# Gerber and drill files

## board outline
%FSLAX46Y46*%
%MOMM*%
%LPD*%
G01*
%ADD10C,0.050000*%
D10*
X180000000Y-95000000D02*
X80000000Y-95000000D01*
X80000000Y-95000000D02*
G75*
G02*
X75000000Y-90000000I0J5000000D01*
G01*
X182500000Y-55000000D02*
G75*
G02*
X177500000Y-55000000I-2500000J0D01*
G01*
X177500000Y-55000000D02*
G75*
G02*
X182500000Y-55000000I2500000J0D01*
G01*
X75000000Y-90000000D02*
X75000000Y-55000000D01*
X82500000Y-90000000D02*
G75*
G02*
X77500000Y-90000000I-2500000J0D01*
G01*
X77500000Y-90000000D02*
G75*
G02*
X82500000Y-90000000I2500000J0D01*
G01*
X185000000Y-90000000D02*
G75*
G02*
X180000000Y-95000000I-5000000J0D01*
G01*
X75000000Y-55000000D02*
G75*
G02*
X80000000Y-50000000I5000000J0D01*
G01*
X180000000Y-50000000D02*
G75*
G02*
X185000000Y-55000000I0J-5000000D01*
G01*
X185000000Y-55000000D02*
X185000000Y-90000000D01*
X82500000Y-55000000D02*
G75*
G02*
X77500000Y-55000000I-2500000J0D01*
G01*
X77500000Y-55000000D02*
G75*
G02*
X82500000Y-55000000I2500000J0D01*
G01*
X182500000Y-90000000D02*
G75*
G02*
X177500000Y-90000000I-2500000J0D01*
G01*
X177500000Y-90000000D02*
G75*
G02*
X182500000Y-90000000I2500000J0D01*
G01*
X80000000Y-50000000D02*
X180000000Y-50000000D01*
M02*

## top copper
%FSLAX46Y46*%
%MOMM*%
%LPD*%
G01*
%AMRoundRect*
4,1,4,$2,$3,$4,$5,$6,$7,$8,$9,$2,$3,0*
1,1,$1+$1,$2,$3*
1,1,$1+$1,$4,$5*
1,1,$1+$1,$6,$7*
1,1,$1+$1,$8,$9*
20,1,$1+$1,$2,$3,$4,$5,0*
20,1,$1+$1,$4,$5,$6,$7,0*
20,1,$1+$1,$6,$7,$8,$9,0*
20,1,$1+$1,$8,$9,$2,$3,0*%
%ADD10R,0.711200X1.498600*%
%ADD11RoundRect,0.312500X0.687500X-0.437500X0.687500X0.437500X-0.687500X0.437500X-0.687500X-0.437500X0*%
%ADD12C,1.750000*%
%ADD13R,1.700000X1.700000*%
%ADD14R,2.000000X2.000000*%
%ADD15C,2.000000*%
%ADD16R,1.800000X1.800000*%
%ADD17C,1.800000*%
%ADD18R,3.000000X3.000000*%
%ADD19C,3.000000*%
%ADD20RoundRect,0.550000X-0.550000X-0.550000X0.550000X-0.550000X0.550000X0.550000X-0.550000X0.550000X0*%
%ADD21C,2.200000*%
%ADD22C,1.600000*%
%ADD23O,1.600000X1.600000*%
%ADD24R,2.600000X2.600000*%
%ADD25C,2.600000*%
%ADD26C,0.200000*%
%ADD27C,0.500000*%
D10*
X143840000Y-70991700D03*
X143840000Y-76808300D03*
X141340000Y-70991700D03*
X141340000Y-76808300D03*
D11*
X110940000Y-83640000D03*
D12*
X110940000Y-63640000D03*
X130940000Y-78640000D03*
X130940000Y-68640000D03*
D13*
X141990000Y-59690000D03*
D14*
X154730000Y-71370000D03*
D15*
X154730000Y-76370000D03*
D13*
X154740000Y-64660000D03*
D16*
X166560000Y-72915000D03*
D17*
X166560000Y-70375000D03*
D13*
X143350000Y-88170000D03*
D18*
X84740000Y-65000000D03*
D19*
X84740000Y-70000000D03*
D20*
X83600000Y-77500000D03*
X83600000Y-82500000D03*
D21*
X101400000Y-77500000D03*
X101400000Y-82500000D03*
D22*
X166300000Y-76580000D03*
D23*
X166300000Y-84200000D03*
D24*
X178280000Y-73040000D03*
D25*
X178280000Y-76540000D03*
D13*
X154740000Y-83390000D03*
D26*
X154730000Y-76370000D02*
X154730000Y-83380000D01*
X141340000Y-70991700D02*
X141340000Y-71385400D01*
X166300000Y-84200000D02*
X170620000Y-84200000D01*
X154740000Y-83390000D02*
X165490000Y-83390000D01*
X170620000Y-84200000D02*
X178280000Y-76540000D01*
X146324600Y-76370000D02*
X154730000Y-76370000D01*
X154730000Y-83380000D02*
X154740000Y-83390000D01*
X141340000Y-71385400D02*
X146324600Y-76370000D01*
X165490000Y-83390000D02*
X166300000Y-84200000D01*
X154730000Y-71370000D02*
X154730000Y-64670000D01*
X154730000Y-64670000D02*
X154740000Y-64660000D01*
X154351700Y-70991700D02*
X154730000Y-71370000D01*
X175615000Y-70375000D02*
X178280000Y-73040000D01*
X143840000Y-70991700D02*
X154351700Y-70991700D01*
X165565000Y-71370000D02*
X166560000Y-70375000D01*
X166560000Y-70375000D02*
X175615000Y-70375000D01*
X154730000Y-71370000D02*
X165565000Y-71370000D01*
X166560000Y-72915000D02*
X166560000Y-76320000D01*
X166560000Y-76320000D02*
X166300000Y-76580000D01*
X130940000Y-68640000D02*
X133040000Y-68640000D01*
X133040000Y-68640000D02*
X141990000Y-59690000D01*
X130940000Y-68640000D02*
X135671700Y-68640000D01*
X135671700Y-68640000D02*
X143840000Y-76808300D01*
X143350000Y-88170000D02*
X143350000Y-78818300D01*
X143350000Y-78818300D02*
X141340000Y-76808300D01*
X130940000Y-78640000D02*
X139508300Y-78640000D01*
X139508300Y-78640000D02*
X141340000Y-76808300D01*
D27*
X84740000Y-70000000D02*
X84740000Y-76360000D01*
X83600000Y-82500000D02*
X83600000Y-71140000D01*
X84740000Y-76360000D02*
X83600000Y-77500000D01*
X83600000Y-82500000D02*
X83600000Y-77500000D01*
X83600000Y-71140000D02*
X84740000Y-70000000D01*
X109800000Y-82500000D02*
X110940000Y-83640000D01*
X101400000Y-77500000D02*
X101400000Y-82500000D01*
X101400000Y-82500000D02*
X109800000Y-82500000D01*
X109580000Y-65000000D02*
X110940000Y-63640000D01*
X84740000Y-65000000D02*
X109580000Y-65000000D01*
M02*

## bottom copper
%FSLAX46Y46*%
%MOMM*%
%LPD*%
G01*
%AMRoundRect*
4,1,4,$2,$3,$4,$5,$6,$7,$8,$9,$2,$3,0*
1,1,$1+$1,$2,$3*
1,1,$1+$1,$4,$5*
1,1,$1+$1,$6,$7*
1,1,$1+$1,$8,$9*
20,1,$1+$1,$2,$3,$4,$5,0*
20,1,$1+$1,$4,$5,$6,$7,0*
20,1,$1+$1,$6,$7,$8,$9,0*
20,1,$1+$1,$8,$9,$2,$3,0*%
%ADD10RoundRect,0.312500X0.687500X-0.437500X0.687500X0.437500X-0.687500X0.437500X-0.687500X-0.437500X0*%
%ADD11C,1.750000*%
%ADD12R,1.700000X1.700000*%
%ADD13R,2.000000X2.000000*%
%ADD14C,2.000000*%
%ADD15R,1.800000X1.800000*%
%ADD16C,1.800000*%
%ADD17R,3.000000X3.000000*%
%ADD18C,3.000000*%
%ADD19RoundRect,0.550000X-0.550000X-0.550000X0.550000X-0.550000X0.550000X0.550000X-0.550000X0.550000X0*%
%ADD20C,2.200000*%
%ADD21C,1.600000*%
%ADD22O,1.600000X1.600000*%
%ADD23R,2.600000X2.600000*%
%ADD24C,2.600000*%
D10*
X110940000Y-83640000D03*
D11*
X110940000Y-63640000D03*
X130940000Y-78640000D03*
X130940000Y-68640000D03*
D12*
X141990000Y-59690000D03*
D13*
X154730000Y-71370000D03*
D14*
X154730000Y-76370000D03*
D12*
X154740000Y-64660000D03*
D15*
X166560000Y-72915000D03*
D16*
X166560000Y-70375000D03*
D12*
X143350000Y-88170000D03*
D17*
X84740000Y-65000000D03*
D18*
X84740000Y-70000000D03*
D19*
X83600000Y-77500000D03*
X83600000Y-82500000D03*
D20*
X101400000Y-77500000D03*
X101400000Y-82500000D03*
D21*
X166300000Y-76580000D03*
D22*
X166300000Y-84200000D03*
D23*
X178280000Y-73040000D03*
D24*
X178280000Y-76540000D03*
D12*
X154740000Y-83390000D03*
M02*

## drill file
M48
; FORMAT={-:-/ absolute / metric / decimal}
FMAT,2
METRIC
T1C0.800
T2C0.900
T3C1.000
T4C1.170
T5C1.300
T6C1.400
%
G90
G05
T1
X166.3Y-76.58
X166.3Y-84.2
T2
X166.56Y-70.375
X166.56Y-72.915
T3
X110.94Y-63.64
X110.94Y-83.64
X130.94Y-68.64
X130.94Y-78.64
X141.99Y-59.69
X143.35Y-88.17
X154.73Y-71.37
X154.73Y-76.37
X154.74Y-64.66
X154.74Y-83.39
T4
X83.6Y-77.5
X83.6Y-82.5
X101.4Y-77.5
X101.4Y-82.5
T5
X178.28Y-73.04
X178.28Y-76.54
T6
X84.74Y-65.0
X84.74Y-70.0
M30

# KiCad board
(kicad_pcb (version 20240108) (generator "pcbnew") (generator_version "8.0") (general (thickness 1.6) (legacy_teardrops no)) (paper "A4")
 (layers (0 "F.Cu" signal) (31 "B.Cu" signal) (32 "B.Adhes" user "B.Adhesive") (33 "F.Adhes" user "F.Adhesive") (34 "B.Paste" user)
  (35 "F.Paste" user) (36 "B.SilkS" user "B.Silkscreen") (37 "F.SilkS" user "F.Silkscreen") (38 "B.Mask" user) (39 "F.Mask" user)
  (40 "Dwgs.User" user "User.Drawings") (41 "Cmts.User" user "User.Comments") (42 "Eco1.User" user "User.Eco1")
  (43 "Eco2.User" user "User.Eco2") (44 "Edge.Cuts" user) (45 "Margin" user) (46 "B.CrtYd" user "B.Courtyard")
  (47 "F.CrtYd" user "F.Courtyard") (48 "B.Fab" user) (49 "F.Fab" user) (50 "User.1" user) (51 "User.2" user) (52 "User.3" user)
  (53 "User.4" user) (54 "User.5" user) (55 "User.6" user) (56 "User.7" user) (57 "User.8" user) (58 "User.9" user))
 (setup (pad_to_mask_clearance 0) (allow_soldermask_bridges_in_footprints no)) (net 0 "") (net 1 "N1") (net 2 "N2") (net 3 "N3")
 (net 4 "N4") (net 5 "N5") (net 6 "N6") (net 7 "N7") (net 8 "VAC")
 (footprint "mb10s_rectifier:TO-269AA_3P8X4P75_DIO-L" (layer "F.Cu") (at 142.59 73.9 -90)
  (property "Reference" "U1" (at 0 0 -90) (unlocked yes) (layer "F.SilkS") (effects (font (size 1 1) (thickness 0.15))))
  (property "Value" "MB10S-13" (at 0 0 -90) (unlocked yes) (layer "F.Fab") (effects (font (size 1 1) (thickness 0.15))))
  (pad "1" smd rect (at -2.9083 -1.25 270) (size 1.4986 0.7112) (layers "F.Cu" "F.Paste" "F.Mask") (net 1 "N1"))
  (pad "2" smd rect (at 2.9083 -1.25 270) (size 1.4986 0.7112) (layers "F.Cu" "F.Paste" "F.Mask") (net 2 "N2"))
  (pad "3" smd rect (at -2.9083 1.25 270) (size 1.4986 0.7112) (layers "F.Cu" "F.Paste" "F.Mask") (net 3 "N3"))
  (pad "4" smd rect (at 2.9083 1.25 270) (size 1.4986 0.7112) (layers "F.Cu" "F.Paste" "F.Mask") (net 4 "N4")))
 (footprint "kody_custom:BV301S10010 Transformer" (layer "F.Cu") (at 105.94 71.14 90)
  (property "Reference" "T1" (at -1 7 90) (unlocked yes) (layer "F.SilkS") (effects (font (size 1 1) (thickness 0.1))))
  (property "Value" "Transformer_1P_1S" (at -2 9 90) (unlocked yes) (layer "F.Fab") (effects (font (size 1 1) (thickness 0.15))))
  (pad "1" thru_hole roundrect (at -12.5 5 90) (size 1.5 2) (drill 1) (layers "*.Cu" "*.Mask") (remove_unused_layers no)
   (roundrect_rratio 0.2083333333) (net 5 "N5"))
  (pad "2" thru_hole circle (at 7.5 5 90) (size 1.75 1.75) (drill 1) (layers "*.Cu" "*.Mask") (remove_unused_layers no) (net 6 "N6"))
  (pad "3" thru_hole circle (at -7.5 25 90) (size 1.75 1.75) (drill 1) (layers "*.Cu" "*.Mask") (remove_unused_layers no) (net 4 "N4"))
  (pad "4" thru_hole circle (at 2.5 25 90) (size 1.75 1.75) (drill 1) (layers "*.Cu" "*.Mask") (remove_unused_layers no) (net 2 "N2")))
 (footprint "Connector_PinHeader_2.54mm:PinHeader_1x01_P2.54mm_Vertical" (layer "F.Cu") (at 141.99 59.69)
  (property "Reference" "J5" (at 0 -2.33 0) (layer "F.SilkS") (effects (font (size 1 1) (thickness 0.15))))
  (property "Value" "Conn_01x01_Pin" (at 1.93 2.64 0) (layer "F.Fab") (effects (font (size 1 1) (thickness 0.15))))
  (pad "1" thru_hole rect (at 0 0) (size 1.7 1.7) (drill 1) (layers "*.Cu" "*.Mask") (remove_unused_layers no) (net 2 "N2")))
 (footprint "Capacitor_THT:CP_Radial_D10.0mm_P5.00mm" (layer "F.Cu") (at 154.73 71.37 -90)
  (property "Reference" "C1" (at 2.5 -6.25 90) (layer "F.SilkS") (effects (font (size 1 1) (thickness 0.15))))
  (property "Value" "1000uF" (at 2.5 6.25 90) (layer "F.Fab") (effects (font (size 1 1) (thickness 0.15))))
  (pad "1" thru_hole rect (at 0 0 270) (size 2 2) (drill 1) (layers "*.Cu" "*.Mask") (remove_unused_layers no) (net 1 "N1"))
  (pad "2" thru_hole circle (at 5 0 270) (size 2 2) (drill 1) (layers "*.Cu" "*.Mask") (remove_unused_layers no) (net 3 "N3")))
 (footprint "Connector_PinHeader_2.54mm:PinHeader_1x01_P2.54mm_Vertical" (layer "F.Cu") (at 154.74 64.66)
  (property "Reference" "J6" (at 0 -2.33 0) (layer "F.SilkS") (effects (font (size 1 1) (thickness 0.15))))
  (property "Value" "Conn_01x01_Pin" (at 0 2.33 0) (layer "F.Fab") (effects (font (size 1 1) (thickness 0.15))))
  (pad "1" thru_hole rect (at 0 0) (size 1.7 1.7) (drill 1) (layers "*.Cu" "*.Mask") (remove_unused_layers no) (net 1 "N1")))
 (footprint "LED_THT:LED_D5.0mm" (layer "F.Cu") (at 166.56 72.915 90)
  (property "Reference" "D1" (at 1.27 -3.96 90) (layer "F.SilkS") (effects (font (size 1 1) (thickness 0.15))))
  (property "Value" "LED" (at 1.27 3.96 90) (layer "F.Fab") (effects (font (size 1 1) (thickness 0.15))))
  (pad "1" thru_hole rect (at 0 0 90) (size 1.8 1.8) (drill 0.9) (layers "*.Cu" "*.Mask") (remove_unused_layers no) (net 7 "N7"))
  (pad "2" thru_hole circle (at 2.54 0 90) (size 1.8 1.8) (drill 0.9) (layers "*.Cu" "*.Mask") (remove_unused_layers no) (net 1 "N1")))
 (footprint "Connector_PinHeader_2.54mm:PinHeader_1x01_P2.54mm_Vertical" (layer "F.Cu") (at 143.35 88.17)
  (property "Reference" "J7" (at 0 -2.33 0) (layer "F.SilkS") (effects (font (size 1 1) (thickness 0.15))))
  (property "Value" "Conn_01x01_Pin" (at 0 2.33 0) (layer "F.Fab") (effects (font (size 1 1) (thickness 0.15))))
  (pad "1" thru_hole rect (at 0 0) (size 1.7 1.7) (drill 1) (layers "*.Cu" "*.Mask") (remove_unused_layers no) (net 4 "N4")))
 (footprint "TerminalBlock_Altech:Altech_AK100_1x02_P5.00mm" (layer "F.Cu") (at 84.74 65 -90)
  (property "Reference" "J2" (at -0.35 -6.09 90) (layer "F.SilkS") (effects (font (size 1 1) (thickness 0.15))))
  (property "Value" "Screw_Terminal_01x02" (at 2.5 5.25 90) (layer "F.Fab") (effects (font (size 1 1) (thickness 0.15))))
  (pad "1" thru_hole rect (at 0 0 270) (size 3 3) (drill 1.4) (layers "*.Cu" "*.Mask") (remove_unused_layers no) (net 6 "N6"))
  (pad "2" thru_hole circle (at 5 0 270) (size 3 3) (drill 1.4) (layers "*.Cu" "*.Mask") (remove_unused_layers no) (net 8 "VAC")))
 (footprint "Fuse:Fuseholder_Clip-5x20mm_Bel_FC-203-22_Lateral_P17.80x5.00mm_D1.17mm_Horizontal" (layer "F.Cu") (at 83.6 77.5)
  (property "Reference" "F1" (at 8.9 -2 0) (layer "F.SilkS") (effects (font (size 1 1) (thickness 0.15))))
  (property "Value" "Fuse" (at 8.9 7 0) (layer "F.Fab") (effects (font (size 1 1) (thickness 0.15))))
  (pad "1" thru_hole roundrect (at 0 0) (size 2.2 2.2) (drill 1.17) (layers "*.Cu" "*.Mask") (remove_unused_layers no)
   (roundrect_rratio 0.25) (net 8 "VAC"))
  (pad "1" thru_hole roundrect (at 0 5) (size 2.2 2.2) (drill 1.17) (layers "*.Cu" "*.Mask") (remove_unused_layers no)
   (roundrect_rratio 0.25) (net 8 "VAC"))
  (pad "2" thru_hole circle (at 17.8 0) (size 2.2 2.2) (drill 1.17) (layers "*.Cu" "*.Mask") (remove_unused_layers no) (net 5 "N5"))
  (pad "2" thru_hole circle (at 17.8 5) (size 2.2 2.2) (drill 1.17) (layers "*.Cu" "*.Mask") (remove_unused_layers no) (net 5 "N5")))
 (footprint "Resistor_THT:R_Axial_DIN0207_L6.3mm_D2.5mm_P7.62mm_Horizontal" (layer "F.Cu") (at 166.3 76.58 -90)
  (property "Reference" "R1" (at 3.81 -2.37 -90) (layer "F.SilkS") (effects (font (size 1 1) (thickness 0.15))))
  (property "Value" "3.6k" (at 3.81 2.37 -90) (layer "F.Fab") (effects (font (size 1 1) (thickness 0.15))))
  (pad "1" thru_hole circle (at 0 0 270) (size 1.6 1.6) (drill 0.8) (layers "*.Cu" "*.Mask") (remove_unused_layers no) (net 7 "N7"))
  (pad "2" thru_hole oval (at 7.62 0 270) (size 1.6 1.6) (drill 0.8) (layers "*.Cu" "*.Mask") (remove_unused_layers no) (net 3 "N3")))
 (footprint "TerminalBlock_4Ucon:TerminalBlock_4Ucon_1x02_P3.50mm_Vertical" (layer "F.Cu") (at 178.28 73.04 -90)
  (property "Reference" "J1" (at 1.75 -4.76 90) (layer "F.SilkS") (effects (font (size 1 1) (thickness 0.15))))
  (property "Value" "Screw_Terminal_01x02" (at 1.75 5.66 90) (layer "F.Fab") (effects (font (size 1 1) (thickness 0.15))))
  (pad "1" thru_hole rect (at 0 0 270) (size 2.6 2.6) (drill 1.3) (layers "*.Cu" "*.Mask") (remove_unused_layers no) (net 1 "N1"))
  (pad "2" thru_hole circle (at 3.5 0 270) (size 2.6 2.6) (drill 1.3) (layers "*.Cu" "*.Mask") (remove_unused_layers no) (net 3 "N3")))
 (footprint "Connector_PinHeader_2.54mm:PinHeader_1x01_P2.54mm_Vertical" (layer "F.Cu") (at 154.74 83.39)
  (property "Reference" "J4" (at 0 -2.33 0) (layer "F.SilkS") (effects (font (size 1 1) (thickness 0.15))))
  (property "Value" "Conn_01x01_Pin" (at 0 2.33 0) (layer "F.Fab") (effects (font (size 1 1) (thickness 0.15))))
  (pad "1" thru_hole rect (at 0 0) (size 1.7 1.7) (drill 1) (layers "*.Cu" "*.Mask") (remove_unused_layers no) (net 3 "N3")))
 (gr_line (start 180 95) (end 80 95) (stroke (width 0.05) (type default)) (layer "Edge.Cuts"))
 (gr_arc (start 80 95) (mid 76.464466 93.535534) (end 75 90) (stroke (width 0.05) (type default)) (layer "Edge.Cuts"))
 (gr_circle (center 180 55) (end 180 52.5) (stroke (width 0.05) (type default)) (fill none) (layer "Edge.Cuts"))
 (gr_line (start 75 90) (end 75 55) (stroke (width 0.05) (type default)) (layer "Edge.Cuts"))
 (gr_circle (center 80 90) (end 80 92.5) (stroke (width 0.05) (type default)) (fill none) (layer "Edge.Cuts"))
 (gr_arc (start 185 90) (mid 183.535534 93.535534) (end 180 95) (stroke (width 0.05) (type default)) (layer "Edge.Cuts"))
 (gr_arc (start 75 55) (mid 76.464466 51.464466) (end 80 50) (stroke (width 0.05) (type default)) (layer "Edge.Cuts"))
 (gr_arc (start 180 50) (mid 183.535534 51.464466) (end 185 55) (stroke (width 0.05) (type default)) (layer "Edge.Cuts"))
 (gr_line (start 185 55) (end 185 90) (stroke (width 0.05) (type default)) (layer "Edge.Cuts"))
 (gr_circle (center 80 55) (end 77.5 55) (stroke (width 0.05) (type default)) (fill none) (layer "Edge.Cuts"))
 (gr_circle (center 180 90) (end 180 87.5) (stroke (width 0.05) (type default)) (fill none) (layer "Edge.Cuts"))
 (gr_line (start 80 50) (end 180 50) (stroke (width 0.05) (type default)) (layer "Edge.Cuts"))
 (segment (start 154.73 76.37) (end 154.73 83.38) (width 0.2) (layer "F.Cu") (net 3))
 (segment (start 141.34 70.9917) (end 141.34 71.3854) (width 0.2) (layer "F.Cu") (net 3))
 (segment (start 166.3 84.2) (end 170.62 84.2) (width 0.2) (layer "F.Cu") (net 3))
 (segment (start 154.74 83.39) (end 165.49 83.39) (width 0.2) (layer "F.Cu") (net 3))
 (segment (start 170.62 84.2) (end 178.28 76.54) (width 0.2) (layer "F.Cu") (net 3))
 (segment (start 146.3246 76.37) (end 154.73 76.37) (width 0.2) (layer "F.Cu") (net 3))
 (segment (start 154.73 83.38) (end 154.74 83.39) (width 0.2) (layer "F.Cu") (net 3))
 (segment (start 141.34 71.3854) (end 146.3246 76.37) (width 0.2) (layer "F.Cu") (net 3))
 (segment (start 165.49 83.39) (end 166.3 84.2) (width 0.2) (layer "F.Cu") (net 3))
 (segment (start 154.73 71.37) (end 154.73 64.67) (width 0.2) (layer "F.Cu") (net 1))
 (segment (start 154.73 64.67) (end 154.74 64.66) (width 0.2) (layer "F.Cu") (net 1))
 (segment (start 154.3517 70.9917) (end 154.73 71.37) (width 0.2) (layer "F.Cu") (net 1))
 (segment (start 175.615 70.375) (end 178.28 73.04) (width 0.2) (layer "F.Cu") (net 1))
 (segment (start 143.84 70.9917) (end 154.3517 70.9917) (width 0.2) (layer "F.Cu") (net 1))
 (segment (start 165.565 71.37) (end 166.56 70.375) (width 0.2) (layer "F.Cu") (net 1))
 (segment (start 166.56 70.375) (end 175.615 70.375) (width 0.2) (layer "F.Cu") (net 1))
 (segment (start 154.73 71.37) (end 165.565 71.37) (width 0.2) (layer "F.Cu") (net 1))
 (segment (start 166.56 72.915) (end 166.56 76.32) (width 0.2) (layer "F.Cu") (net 7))
 (segment (start 166.56 76.32) (end 166.3 76.58) (width 0.2) (layer "F.Cu") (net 7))
 (segment (start 130.94 68.64) (end 133.04 68.64) (width 0.2) (layer "F.Cu") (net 2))
 (segment (start 133.04 68.64) (end 141.99 59.69) (width 0.2) (layer "F.Cu") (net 2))
 (segment (start 130.94 68.64) (end 135.6717 68.64) (width 0.2) (layer "F.Cu") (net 2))
 (segment (start 135.6717 68.64) (end 143.84 76.8083) (width 0.2) (layer "F.Cu") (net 2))
 (segment (start 143.35 88.17) (end 143.35 78.8183) (width 0.2) (layer "F.Cu") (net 4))
 (segment (start 143.35 78.8183) (end 141.34 76.8083) (width 0.2) (layer "F.Cu") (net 4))
 (segment (start 130.94 78.64) (end 139.5083 78.64) (width 0.2) (layer "F.Cu") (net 4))
 (segment (start 139.5083 78.64) (end 141.34 76.8083) (width 0.2) (layer "F.Cu") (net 4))
 (segment (start 84.74 70) (end 84.74 76.36) (width 0.5) (layer "F.Cu") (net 8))
 (segment (start 83.6 82.5) (end 83.6 71.14) (width 0.5) (layer "F.Cu") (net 8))
 (segment (start 84.74 76.36) (end 83.6 77.5) (width 0.5) (layer "F.Cu") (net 8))
 (segment (start 83.6 82.5) (end 83.6 77.5) (width 0.5) (layer "F.Cu") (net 8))
 (segment (start 83.6 71.14) (end 84.74 70) (width 0.5) (layer "F.Cu") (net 8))
 (segment (start 109.8 82.5) (end 110.94 83.64) (width 0.5) (layer "F.Cu") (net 5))
 (segment (start 101.4 77.5) (end 101.4 82.5) (width 0.5) (layer "F.Cu") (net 5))
 (segment (start 101.4 82.5) (end 109.8 82.5) (width 0.5) (layer "F.Cu") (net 5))
 (segment (start 109.58 65) (end 110.94 63.64) (width 0.5) (layer "F.Cu") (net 6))
 (segment (start 84.74 65) (end 109.58 65) (width 0.5) (layer "F.Cu") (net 6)))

